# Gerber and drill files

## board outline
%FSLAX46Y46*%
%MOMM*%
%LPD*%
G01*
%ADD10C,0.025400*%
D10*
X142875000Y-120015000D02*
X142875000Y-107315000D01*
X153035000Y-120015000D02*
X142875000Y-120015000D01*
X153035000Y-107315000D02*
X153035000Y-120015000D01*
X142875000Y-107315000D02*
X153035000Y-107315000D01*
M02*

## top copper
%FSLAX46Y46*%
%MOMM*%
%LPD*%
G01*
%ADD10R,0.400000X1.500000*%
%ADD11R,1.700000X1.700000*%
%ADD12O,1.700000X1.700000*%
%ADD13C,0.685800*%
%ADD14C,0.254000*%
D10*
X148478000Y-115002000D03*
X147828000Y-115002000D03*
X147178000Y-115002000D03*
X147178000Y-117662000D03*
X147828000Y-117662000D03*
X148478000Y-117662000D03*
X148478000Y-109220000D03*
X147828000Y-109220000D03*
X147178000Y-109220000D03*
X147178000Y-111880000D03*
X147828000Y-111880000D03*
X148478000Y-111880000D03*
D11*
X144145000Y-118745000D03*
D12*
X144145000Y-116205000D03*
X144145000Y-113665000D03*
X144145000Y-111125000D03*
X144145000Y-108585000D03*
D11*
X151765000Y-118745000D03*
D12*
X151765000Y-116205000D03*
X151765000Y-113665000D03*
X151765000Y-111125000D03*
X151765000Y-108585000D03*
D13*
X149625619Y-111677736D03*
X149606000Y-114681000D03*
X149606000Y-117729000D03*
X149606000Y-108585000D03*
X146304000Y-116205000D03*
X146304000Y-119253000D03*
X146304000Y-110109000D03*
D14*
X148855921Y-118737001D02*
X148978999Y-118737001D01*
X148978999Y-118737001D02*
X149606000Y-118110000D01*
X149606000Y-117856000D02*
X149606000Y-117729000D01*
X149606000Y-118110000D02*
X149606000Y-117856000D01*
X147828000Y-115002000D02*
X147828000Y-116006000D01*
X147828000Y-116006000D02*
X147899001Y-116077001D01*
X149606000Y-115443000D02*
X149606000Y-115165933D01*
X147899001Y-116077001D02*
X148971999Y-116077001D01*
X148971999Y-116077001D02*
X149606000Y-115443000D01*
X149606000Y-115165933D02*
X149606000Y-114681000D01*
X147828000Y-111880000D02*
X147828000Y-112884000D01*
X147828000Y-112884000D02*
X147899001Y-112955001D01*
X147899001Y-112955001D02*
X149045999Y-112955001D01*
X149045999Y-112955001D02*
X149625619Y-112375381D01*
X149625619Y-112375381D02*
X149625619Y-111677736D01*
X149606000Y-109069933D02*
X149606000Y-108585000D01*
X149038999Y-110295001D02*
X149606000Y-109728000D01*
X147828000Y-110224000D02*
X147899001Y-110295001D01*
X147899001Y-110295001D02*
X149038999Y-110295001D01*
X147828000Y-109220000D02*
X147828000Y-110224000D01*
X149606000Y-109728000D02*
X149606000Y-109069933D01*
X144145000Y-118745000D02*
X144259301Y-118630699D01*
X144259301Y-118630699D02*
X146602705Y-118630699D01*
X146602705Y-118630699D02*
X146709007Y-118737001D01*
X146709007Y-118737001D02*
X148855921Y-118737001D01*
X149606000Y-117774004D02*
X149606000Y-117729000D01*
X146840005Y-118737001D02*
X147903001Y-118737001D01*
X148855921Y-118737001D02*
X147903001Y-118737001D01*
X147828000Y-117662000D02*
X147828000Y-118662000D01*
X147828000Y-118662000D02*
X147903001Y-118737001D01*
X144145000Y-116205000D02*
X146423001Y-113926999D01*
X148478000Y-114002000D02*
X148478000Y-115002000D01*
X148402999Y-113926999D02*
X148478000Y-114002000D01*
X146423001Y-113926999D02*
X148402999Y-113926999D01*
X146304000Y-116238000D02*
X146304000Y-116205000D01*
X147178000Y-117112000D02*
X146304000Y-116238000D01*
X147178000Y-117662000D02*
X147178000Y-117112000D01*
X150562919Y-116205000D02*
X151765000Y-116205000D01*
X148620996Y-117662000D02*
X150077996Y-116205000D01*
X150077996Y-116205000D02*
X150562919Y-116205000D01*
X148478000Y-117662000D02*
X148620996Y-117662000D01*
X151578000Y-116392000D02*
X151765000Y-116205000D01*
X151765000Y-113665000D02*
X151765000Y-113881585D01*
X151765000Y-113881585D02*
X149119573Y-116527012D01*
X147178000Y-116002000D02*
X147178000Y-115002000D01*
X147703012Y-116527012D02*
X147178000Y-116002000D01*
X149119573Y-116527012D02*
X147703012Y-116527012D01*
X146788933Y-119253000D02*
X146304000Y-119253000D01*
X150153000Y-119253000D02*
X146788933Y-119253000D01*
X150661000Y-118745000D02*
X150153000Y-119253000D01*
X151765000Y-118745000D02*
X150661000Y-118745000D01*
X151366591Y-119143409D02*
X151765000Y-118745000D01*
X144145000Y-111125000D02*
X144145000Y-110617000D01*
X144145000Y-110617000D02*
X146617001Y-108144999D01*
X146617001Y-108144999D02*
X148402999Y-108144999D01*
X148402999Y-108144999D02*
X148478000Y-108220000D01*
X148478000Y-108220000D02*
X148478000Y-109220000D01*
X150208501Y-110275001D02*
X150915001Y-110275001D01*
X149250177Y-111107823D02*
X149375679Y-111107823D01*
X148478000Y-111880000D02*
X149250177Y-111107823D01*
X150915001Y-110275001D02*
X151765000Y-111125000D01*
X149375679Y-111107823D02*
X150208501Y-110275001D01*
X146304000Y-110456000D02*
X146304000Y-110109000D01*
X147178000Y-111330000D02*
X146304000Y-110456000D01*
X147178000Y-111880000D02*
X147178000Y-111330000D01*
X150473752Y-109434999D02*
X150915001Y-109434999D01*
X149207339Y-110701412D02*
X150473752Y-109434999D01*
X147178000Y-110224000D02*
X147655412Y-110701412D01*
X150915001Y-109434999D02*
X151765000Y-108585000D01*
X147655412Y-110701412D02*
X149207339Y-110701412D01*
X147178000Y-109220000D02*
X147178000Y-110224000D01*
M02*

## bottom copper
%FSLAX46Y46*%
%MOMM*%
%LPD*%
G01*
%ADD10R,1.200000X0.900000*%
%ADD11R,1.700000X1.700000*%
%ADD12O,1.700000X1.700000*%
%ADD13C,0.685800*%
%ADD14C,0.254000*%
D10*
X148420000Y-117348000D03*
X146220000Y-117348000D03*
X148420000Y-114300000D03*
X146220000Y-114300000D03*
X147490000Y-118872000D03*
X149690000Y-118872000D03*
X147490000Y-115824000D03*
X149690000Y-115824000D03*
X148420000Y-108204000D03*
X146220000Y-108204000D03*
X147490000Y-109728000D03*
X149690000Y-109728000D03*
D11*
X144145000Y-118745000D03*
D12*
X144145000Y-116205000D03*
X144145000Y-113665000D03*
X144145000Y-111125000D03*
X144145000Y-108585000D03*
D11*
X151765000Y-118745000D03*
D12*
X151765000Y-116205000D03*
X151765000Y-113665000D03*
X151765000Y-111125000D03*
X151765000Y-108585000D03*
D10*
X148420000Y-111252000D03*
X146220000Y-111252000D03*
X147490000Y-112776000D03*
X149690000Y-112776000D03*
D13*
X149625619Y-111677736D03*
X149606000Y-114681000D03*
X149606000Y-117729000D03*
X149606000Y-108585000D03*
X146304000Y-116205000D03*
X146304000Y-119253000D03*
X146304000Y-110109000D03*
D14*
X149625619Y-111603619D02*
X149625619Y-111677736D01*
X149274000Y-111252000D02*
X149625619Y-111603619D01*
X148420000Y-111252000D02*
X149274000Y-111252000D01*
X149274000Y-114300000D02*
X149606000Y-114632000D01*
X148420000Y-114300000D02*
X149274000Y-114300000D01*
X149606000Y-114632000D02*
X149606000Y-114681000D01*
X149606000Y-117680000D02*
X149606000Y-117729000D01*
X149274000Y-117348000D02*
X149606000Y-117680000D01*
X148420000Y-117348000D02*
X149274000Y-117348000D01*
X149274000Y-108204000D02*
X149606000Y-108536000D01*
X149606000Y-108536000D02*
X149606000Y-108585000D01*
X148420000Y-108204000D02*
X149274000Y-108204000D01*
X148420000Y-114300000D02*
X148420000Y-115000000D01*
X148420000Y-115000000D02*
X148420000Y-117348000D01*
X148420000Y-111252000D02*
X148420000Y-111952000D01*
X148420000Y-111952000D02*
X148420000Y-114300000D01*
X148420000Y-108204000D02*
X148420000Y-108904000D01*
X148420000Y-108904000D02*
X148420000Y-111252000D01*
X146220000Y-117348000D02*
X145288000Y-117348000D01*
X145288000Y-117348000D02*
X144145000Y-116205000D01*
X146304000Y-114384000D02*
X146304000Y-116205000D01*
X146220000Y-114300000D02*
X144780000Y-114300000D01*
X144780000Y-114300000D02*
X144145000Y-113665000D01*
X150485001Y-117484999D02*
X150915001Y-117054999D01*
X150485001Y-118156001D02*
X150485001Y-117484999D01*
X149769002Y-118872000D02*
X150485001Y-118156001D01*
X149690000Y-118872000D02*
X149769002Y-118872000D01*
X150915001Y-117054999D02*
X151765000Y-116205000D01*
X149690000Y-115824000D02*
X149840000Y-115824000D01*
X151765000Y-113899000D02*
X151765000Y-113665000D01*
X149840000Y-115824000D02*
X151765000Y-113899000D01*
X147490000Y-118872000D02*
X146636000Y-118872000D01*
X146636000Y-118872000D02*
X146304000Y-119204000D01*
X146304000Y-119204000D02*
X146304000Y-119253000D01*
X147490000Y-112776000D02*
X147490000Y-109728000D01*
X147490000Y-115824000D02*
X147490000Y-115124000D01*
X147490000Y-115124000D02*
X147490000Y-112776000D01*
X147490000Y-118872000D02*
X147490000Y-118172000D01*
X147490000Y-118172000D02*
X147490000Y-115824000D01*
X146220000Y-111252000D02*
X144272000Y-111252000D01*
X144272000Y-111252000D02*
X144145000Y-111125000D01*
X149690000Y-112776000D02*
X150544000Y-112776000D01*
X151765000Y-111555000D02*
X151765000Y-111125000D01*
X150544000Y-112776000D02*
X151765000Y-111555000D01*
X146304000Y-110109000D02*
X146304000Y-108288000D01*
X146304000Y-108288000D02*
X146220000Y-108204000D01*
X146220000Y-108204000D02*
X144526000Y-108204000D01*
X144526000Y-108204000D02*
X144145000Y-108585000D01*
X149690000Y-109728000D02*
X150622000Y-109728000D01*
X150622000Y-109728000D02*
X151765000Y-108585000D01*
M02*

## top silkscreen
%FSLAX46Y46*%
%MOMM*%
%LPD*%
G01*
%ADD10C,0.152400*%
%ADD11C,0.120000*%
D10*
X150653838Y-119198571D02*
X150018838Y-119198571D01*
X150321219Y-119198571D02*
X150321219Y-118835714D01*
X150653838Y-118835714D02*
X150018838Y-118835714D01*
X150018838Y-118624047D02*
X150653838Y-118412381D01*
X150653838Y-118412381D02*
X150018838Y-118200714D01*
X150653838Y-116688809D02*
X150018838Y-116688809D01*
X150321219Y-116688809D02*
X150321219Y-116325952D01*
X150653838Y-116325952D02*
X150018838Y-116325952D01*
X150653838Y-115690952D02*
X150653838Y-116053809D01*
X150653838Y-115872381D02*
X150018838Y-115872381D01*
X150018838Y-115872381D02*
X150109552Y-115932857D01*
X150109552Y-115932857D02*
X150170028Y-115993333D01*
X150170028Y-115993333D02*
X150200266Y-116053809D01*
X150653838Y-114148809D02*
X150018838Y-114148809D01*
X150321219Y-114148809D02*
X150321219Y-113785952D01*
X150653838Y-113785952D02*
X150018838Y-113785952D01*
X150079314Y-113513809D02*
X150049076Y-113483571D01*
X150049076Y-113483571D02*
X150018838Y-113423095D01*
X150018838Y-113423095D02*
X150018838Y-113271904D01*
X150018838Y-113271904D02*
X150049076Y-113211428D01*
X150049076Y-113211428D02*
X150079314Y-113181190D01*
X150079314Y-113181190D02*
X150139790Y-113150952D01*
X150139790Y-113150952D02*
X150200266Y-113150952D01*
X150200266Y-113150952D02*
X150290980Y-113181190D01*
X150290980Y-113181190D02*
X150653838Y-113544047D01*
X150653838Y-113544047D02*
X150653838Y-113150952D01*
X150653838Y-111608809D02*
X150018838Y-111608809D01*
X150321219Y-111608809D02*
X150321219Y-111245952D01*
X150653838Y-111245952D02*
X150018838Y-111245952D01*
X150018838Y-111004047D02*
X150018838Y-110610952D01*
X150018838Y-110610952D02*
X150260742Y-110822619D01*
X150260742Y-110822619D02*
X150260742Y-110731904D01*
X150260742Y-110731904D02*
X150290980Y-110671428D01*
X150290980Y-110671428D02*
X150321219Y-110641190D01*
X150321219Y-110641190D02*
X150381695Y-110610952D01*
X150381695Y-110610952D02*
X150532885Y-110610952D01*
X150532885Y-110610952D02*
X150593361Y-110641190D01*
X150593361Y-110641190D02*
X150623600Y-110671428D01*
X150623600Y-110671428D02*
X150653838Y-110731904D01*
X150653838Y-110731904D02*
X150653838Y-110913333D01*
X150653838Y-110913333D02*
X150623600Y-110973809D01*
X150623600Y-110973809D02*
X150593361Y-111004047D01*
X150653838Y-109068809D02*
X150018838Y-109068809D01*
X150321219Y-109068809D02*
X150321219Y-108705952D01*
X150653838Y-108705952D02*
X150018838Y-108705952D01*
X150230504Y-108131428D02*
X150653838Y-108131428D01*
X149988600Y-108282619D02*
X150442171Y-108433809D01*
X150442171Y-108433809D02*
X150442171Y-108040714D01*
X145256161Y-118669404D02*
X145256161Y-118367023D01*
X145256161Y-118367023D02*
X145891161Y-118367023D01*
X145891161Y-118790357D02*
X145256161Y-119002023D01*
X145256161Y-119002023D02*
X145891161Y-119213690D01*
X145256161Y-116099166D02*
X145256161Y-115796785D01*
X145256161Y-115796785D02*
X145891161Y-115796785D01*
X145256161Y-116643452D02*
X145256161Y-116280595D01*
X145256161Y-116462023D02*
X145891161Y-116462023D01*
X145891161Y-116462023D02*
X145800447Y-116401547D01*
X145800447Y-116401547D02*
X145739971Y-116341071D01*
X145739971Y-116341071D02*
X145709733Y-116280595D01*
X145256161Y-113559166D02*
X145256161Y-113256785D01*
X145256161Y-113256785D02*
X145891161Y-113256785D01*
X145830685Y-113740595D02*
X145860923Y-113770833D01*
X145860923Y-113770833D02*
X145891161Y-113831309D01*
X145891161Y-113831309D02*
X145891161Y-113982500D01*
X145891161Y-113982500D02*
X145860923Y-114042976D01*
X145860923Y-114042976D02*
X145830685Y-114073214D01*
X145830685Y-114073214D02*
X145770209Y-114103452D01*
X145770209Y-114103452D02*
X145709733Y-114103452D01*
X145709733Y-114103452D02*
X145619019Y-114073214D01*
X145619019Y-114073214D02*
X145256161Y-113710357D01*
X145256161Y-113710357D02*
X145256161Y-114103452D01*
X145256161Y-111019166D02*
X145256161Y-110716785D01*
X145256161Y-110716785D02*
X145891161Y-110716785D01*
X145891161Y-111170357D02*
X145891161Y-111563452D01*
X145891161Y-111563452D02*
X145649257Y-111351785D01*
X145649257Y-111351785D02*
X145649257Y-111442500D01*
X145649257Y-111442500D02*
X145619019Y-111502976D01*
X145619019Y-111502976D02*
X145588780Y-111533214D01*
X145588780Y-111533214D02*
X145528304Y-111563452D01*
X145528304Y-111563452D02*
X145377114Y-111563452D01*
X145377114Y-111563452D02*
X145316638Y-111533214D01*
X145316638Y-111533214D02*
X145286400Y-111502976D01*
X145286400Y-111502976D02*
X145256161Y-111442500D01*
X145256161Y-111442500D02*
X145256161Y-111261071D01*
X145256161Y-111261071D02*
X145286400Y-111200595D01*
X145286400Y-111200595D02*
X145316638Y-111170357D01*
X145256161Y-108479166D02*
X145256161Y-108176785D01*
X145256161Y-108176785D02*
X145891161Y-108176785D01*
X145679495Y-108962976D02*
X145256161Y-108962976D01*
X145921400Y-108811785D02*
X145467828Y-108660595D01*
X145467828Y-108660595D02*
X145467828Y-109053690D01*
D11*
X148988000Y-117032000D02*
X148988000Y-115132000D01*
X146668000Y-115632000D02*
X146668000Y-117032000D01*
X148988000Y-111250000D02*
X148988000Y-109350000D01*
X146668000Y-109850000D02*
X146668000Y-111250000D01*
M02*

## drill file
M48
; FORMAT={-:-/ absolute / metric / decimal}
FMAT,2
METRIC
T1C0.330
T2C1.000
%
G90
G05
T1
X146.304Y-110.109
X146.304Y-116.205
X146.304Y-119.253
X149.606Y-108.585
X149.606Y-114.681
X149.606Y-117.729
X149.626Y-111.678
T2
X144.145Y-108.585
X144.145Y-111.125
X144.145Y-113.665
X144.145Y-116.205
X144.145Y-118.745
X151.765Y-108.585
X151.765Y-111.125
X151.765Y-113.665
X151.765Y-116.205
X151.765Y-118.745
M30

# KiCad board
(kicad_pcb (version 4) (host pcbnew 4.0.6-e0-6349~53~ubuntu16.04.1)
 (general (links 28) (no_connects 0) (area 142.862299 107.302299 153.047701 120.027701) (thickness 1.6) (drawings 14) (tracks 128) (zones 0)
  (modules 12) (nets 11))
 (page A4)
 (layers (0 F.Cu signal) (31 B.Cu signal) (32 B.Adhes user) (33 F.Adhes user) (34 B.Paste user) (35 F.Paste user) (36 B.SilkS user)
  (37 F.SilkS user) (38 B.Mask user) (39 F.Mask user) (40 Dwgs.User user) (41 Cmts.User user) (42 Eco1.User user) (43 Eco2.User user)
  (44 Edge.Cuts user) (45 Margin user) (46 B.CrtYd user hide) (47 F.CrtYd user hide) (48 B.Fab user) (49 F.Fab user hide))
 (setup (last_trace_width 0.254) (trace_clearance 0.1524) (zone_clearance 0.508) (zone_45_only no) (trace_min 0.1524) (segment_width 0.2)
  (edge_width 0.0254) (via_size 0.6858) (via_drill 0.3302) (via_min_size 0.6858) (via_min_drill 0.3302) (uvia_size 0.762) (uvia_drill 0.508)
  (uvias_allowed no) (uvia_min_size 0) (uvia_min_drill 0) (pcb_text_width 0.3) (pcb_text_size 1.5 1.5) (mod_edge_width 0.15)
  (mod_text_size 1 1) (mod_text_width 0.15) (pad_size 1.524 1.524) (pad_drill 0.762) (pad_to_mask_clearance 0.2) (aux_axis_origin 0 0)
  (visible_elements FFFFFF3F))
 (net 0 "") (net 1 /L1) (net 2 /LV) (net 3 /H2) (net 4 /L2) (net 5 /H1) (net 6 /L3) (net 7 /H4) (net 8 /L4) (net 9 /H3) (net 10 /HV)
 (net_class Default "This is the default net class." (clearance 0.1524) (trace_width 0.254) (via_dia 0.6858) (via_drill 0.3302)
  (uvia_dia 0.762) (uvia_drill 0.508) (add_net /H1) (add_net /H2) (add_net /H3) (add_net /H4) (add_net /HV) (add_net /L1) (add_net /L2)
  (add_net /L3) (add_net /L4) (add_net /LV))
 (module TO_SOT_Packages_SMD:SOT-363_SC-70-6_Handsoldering (layer F.Cu) (at 147.828 116.332 270)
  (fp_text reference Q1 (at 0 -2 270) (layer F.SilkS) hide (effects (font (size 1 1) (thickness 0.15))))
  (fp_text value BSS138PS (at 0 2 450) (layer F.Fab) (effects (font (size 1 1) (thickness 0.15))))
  (fp_line (start 0.7 -1.16) (end -1.2 -1.16) (layer F.SilkS) (width 0.12))
  (fp_line (start -0.7 1.16) (end 0.7 1.16) (layer F.SilkS) (width 0.12))
  (pad 1 smd rect (at -1.33 -0.65 270) (size 1.5 0.4) (layers F.Cu F.Paste F.Mask) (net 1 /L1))
  (pad 2 smd rect (at -1.33 0 270) (size 1.5 0.4) (layers F.Cu F.Paste F.Mask) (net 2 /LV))
  (pad 3 smd rect (at -1.33 0.65 270) (size 1.5 0.4) (layers F.Cu F.Paste F.Mask) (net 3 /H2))
  (pad 4 smd rect (at 1.33 0.65 270) (size 1.5 0.4) (layers F.Cu F.Paste F.Mask) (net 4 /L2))
  (pad 5 smd rect (at 1.33 0 270) (size 1.5 0.4) (layers F.Cu F.Paste F.Mask) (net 2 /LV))
  (pad 6 smd rect (at 1.33 -0.65 270) (size 1.5 0.4) (layers F.Cu F.Paste F.Mask) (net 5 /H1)))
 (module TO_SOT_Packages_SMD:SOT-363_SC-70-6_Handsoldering (layer F.Cu) (at 147.828 110.55 270)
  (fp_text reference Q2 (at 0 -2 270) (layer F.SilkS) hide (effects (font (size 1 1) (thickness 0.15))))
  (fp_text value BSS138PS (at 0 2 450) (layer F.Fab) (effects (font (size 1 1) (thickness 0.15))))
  (fp_line (start 0.7 -1.16) (end -1.2 -1.16) (layer F.SilkS) (width 0.12))
  (fp_line (start -0.7 1.16) (end 0.7 1.16) (layer F.SilkS) (width 0.12))
  (pad 1 smd rect (at -1.33 -0.65 270) (size 1.5 0.4) (layers F.Cu F.Paste F.Mask) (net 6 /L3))
  (pad 2 smd rect (at -1.33 0 270) (size 1.5 0.4) (layers F.Cu F.Paste F.Mask) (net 2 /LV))
  (pad 3 smd rect (at -1.33 0.65 270) (size 1.5 0.4) (layers F.Cu F.Paste F.Mask) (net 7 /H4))
  (pad 4 smd rect (at 1.33 0.65 270) (size 1.5 0.4) (layers F.Cu F.Paste F.Mask) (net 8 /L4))
  (pad 5 smd rect (at 1.33 0 270) (size 1.5 0.4) (layers F.Cu F.Paste F.Mask) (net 2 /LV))
  (pad 6 smd rect (at 1.33 -0.65 270) (size 1.5 0.4) (layers F.Cu F.Paste F.Mask) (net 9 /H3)))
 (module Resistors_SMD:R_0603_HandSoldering (layer B.Cu) (at 147.32 117.348 180)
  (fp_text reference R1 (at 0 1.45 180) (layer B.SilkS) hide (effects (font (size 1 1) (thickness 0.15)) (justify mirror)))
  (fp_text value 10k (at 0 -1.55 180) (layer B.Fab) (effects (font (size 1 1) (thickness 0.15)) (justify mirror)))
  (pad 1 smd rect (at -1.1 0 180) (size 1.2 0.9) (layers B.Cu B.Paste B.Mask) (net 2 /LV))
  (pad 2 smd rect (at 1.1 0 180) (size 1.2 0.9) (layers B.Cu B.Paste B.Mask) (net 1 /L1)))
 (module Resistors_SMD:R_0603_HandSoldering (layer B.Cu) (at 147.32 114.3 180)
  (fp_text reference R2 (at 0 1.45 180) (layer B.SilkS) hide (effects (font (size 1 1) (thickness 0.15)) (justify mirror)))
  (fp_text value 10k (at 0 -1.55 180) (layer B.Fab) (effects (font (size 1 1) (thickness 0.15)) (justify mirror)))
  (pad 1 smd rect (at -1.1 0 180) (size 1.2 0.9) (layers B.Cu B.Paste B.Mask) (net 2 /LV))
  (pad 2 smd rect (at 1.1 0 180) (size 1.2 0.9) (layers B.Cu B.Paste B.Mask) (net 4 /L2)))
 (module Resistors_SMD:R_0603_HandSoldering (layer B.Cu) (at 148.59 118.872)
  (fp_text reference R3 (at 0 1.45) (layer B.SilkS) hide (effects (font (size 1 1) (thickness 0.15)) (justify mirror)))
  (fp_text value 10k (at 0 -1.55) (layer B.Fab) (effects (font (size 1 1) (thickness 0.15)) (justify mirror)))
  (pad 1 smd rect (at -1.1 0) (size 1.2 0.9) (layers B.Cu B.Paste B.Mask) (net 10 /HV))
  (pad 2 smd rect (at 1.1 0) (size 1.2 0.9) (layers B.Cu B.Paste B.Mask) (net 5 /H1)))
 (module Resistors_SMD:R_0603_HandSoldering (layer B.Cu) (at 148.59 115.824)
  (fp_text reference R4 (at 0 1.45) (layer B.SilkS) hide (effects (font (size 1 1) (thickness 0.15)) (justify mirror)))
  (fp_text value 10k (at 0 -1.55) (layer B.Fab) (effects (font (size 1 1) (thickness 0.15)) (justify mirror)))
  (pad 1 smd rect (at -1.1 0) (size 1.2 0.9) (layers B.Cu B.Paste B.Mask) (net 10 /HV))
  (pad 2 smd rect (at 1.1 0) (size 1.2 0.9) (layers B.Cu B.Paste B.Mask) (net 3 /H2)))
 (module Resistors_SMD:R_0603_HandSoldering (layer B.Cu) (at 147.32 108.204 180)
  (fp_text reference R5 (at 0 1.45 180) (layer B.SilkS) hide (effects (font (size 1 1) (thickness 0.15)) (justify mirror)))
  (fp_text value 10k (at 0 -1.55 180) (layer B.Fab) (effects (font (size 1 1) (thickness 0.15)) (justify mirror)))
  (pad 1 smd rect (at -1.1 0 180) (size 1.2 0.9) (layers B.Cu B.Paste B.Mask) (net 2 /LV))
  (pad 2 smd rect (at 1.1 0 180) (size 1.2 0.9) (layers B.Cu B.Paste B.Mask) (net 8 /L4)))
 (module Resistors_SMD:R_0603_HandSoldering (layer B.Cu) (at 148.59 109.728)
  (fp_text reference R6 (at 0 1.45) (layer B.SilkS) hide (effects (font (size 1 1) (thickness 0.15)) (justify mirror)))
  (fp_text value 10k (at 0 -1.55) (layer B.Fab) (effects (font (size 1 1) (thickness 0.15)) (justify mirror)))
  (pad 1 smd rect (at -1.1 0) (size 1.2 0.9) (layers B.Cu B.Paste B.Mask) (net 10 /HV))
  (pad 2 smd rect (at 1.1 0) (size 1.2 0.9) (layers B.Cu B.Paste B.Mask) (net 7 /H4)))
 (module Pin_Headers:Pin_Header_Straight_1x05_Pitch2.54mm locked (layer B.Cu) (at 144.145 118.745)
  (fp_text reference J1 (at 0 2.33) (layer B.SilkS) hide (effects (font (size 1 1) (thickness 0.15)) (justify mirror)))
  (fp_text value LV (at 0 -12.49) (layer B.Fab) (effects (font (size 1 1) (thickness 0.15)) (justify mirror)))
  (pad 1 thru_hole rect (at 0 0) (size 1.7 1.7) (drill 1) (layers *.Cu *.Mask) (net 2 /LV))
  (pad 2 thru_hole oval (at 0 -2.54) (size 1.7 1.7) (drill 1) (layers *.Cu *.Mask) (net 1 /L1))
  (pad 3 thru_hole oval (at 0 -5.08) (size 1.7 1.7) (drill 1) (layers *.Cu *.Mask) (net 4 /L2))
  (pad 4 thru_hole oval (at 0 -7.62) (size 1.7 1.7) (drill 1) (layers *.Cu *.Mask) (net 6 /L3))
  (pad 5 thru_hole oval (at 0 -10.16) (size 1.7 1.7) (drill 1) (layers *.Cu *.Mask) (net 8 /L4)))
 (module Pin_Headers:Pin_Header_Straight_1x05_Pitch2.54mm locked (layer B.Cu) (at 151.765 118.745)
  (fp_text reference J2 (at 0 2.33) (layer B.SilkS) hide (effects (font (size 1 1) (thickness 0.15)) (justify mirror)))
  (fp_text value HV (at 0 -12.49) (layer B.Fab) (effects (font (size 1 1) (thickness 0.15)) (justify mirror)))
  (pad 1 thru_hole rect (at 0 0) (size 1.7 1.7) (drill 1) (layers *.Cu *.Mask) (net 10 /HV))
  (pad 2 thru_hole oval (at 0 -2.54) (size 1.7 1.7) (drill 1) (layers *.Cu *.Mask) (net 5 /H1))
  (pad 3 thru_hole oval (at 0 -5.08) (size 1.7 1.7) (drill 1) (layers *.Cu *.Mask) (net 3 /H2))
  (pad 4 thru_hole oval (at 0 -7.62) (size 1.7 1.7) (drill 1) (layers *.Cu *.Mask) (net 9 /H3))
  (pad 5 thru_hole oval (at 0 -10.16) (size 1.7 1.7) (drill 1) (layers *.Cu *.Mask) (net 7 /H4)))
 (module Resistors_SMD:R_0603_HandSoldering (layer B.Cu) (at 147.32 111.252 180)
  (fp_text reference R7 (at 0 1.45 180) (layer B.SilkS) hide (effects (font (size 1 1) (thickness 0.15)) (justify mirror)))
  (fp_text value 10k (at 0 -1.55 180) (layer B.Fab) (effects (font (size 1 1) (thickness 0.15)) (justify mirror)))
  (pad 1 smd rect (at -1.1 0 180) (size 1.2 0.9) (layers B.Cu B.Paste B.Mask) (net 2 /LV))
  (pad 2 smd rect (at 1.1 0 180) (size 1.2 0.9) (layers B.Cu B.Paste B.Mask) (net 6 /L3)))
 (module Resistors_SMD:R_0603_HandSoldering (layer B.Cu) (at 148.59 112.776)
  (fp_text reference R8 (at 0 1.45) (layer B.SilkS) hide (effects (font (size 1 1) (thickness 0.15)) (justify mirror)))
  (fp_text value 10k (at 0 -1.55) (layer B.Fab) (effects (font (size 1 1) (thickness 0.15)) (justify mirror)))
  (pad 1 smd rect (at -1.1 0) (size 1.2 0.9) (layers B.Cu B.Paste B.Mask) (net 10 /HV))
  (pad 2 smd rect (at 1.1 0) (size 1.2 0.9) (layers B.Cu B.Paste B.Mask) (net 9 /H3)))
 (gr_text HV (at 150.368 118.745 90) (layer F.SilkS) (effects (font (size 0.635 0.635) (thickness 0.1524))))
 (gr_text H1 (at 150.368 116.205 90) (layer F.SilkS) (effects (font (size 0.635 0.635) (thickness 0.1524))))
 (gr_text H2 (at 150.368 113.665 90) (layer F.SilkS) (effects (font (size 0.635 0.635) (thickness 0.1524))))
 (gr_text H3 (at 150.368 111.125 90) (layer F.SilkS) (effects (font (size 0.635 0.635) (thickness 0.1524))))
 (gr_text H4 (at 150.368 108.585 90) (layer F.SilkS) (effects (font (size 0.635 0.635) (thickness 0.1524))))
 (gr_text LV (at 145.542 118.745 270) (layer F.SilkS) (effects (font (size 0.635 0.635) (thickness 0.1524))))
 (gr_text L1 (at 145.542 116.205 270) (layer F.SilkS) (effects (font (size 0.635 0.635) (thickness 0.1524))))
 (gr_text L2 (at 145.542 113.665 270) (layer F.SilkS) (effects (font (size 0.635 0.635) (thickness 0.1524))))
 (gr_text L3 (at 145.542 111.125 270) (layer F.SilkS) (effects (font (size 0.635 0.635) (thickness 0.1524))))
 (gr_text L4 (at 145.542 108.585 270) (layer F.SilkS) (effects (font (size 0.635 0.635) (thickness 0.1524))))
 (gr_line (start 142.875 120.015) (end 142.875 107.315) (angle 90) (layer Edge.Cuts) (width 0.0254))
 (gr_line (start 153.035 120.015) (end 142.875 120.015) (angle 90) (layer Edge.Cuts) (width 0.0254))
 (gr_line (start 153.035 107.315) (end 153.035 120.015) (angle 90) (layer Edge.Cuts) (width 0.0254))
 (gr_line (start 142.875 107.315) (end 153.035 107.315) (angle 90) (layer Edge.Cuts) (width 0.0254))
 (segment (start 148.855921 118.737001) (end 148.978999 118.737001) (width 0.254) (layer F.Cu) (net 2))
 (segment (start 148.978999 118.737001) (end 149.606 118.11) (width 0.254) (layer F.Cu) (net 2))
 (segment (start 149.606 117.856) (end 149.606 117.729) (width 0.254) (layer F.Cu) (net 2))
 (segment (start 149.606 118.11) (end 149.606 117.856) (width 0.254) (layer F.Cu) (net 2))
 (segment (start 147.828 115.002) (end 147.828 116.006) (width 0.254) (layer F.Cu) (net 2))
 (segment (start 147.828 116.006) (end 147.899001 116.077001) (width 0.254) (layer F.Cu) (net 2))
 (segment (start 149.606 115.443) (end 149.606 115.165933) (width 0.254) (layer F.Cu) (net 2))
 (segment (start 147.899001 116.077001) (end 148.971999 116.077001) (width 0.254) (layer F.Cu) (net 2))
 (segment (start 148.971999 116.077001) (end 149.606 115.443) (width 0.254) (layer F.Cu) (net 2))
 (segment (start 149.606 115.165933) (end 149.606 114.681) (width 0.254) (layer F.Cu) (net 2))
 (segment (start 147.828 111.88) (end 147.828 112.884) (width 0.254) (layer F.Cu) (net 2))
 (segment (start 147.828 112.884) (end 147.899001 112.955001) (width 0.254) (layer F.Cu) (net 2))
 (segment (start 147.899001 112.955001) (end 149.045999 112.955001) (width 0.254) (layer F.Cu) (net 2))
 (segment (start 149.045999 112.955001) (end 149.625619 112.375381) (width 0.254) (layer F.Cu) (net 2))
 (segment (start 149.625619 112.375381) (end 149.625619 111.677736) (width 0.254) (layer F.Cu) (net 2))
 (segment (start 149.625619 111.603619) (end 149.625619 111.677736) (width 0.254) (layer B.Cu) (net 2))
 (segment (start 149.606 109.069933) (end 149.606 108.585) (width 0.254) (layer F.Cu) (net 2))
 (segment (start 149.274 111.252) (end 149.625619 111.603619) (width 0.254) (layer B.Cu) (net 2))
 (segment (start 149.038999 110.295001) (end 149.606 109.728) (width 0.254) (layer F.Cu) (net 2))
 (segment (start 148.42 111.252) (end 149.274 111.252) (width 0.254) (layer B.Cu) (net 2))
 (segment (start 147.828 110.224) (end 147.899001 110.295001) (width 0.254) (layer F.Cu) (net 2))
 (segment (start 147.899001 110.295001) (end 149.038999 110.295001) (width 0.254) (layer F.Cu) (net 2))
 (via (at 149.625619 111.677736) (size 0.6858) (drill 0.3302) (layers F.Cu B.Cu) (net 2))
 (segment (start 147.828 109.22) (end 147.828 110.224) (width 0.254) (layer F.Cu) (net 2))
 (segment (start 149.606 109.728) (end 149.606 109.069933) (width 0.254) (layer F.Cu) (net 2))
 (segment (start 144.145 118.745) (end 144.259301 118.630699) (width 0.254) (layer F.Cu) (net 2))
 (segment (start 144.259301 118.630699) (end 146.602705 118.630699) (width 0.254) (layer F.Cu) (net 2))
 (segment (start 146.602705 118.630699) (end 146.709007 118.737001) (width 0.254) (layer F.Cu) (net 2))
 (segment (start 146.709007 118.737001) (end 148.855921 118.737001) (width 0.254) (layer F.Cu) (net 2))
 (segment (start 149.274 114.3) (end 149.606 114.632) (width 0.254) (layer B.Cu) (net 2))
 (segment (start 148.42 114.3) (end 149.274 114.3) (width 0.254) (layer B.Cu) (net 2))
 (segment (start 149.606 114.632) (end 149.606 114.681) (width 0.254) (layer B.Cu) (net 2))
 (via (at 149.606 114.681) (size 0.6858) (drill 0.3302) (layers F.Cu B.Cu) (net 2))
 (segment (start 149.606 117.68) (end 149.606 117.729) (width 0.254) (layer B.Cu) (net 2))
 (segment (start 149.274 117.348) (end 149.606 117.68) (width 0.254) (layer B.Cu) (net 2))
 (segment (start 149.606 117.774004) (end 149.606 117.729) (width 0.254) (layer F.Cu) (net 2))
 (segment (start 148.42 117.348) (end 149.274 117.348) (width 0.254) (layer B.Cu) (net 2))
 (via (at 149.606 117.729) (size 0.6858) (drill 0.3302) (layers F.Cu B.Cu) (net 2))
 (segment (start 149.274 108.204) (end 149.606 108.536) (width 0.254) (layer B.Cu) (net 2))
 (segment (start 149.606 108.536) (end 149.606 108.585) (width 0.254) (layer B.Cu) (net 2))
 (segment (start 148.42 108.204) (end 149.274 108.204) (width 0.254) (layer B.Cu) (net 2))
 (via (at 149.606 108.585) (size 0.6858) (drill 0.3302) (layers F.Cu B.Cu) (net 2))
 (segment (start 146.840005 118.737001) (end 147.903001 118.737001) (width 0.254) (layer F.Cu) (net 2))
 (segment (start 148.855921 118.737001) (end 147.903001 118.737001) (width 0.254) (layer F.Cu) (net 2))
 (segment (start 147.828 117.662) (end 147.828 118.662) (width 0.254) (layer F.Cu) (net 2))
 (segment (start 147.828 118.662) (end 147.903001 118.737001) (width 0.254) (layer F.Cu) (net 2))
 (segment (start 148.42 114.3) (end 148.42 115) (width 0.254) (layer B.Cu) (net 2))
 (segment (start 148.42 115) (end 148.42 117.348) (width 0.254) (layer B.Cu) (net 2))
 (segment (start 148.42 111.252) (end 148.42 111.952) (width 0.254) (layer B.Cu) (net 2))
 (segment (start 148.42 111.952) (end 148.42 114.3) (width 0.254) (layer B.Cu) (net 2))
 (segment (start 148.42 108.204) (end 148.42 108.904) (width 0.254) (layer B.Cu) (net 2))
 (segment (start 148.42 108.904) (end 148.42 111.252) (width 0.254) (layer B.Cu) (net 2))
 (segment (start 144.145 116.205) (end 146.423001 113.926999) (width 0.254) (layer F.Cu) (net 1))
 (segment (start 148.478 114.002) (end 148.478 115.002) (width 0.254) (layer F.Cu) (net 1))
 (segment (start 148.402999 113.926999) (end 148.478 114.002) (width 0.254) (layer F.Cu) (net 1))
 (segment (start 146.423001 113.926999) (end 148.402999 113.926999) (width 0.254) (layer F.Cu) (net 1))
 (segment (start 146.22 117.348) (end 145.288 117.348) (width 0.254) (layer B.Cu) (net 1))
 (segment (start 145.288 117.348) (end 144.145 116.205) (width 0.254) (layer B.Cu) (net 1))
 (segment (start 146.304 116.238) (end 146.304 116.205) (width 0.254) (layer F.Cu) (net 4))
 (segment (start 147.178 117.112) (end 146.304 116.238) (width 0.254) (layer F.Cu) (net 4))
 (segment (start 147.178 117.662) (end 147.178 117.112) (width 0.254) (layer F.Cu) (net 4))
 (segment (start 146.304 114.384) (end 146.304 116.205) (width 0.254) (layer B.Cu) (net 4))
 (via (at 146.304 116.205) (size 0.6858) (drill 0.3302) (layers F.Cu B.Cu) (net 4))
 (segment (start 146.22 114.3) (end 144.78 114.3) (width 0.254) (layer B.Cu) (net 4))
 (segment (start 144.78 114.3) (end 144.145 113.665) (width 0.254) (layer B.Cu) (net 4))
 (segment (start 150.562919 116.205) (end 151.765 116.205) (width 0.254) (layer F.Cu) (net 5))
 (segment (start 148.620996 117.662) (end 150.077996 116.205) (width 0.254) (layer F.Cu) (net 5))
 (segment (start 150.077996 116.205) (end 150.562919 116.205) (width 0.254) (layer F.Cu) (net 5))
 (segment (start 148.478 117.662) (end 148.620996 117.662) (width 0.254) (layer F.Cu) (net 5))
 (segment (start 150.485001 117.484999) (end 150.915001 117.054999) (width 0.254) (layer B.Cu) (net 5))
 (segment (start 150.485001 118.156001) (end 150.485001 117.484999) (width 0.254) (layer B.Cu) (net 5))
 (segment (start 149.769002 118.872) (end 150.485001 118.156001) (width 0.254) (layer B.Cu) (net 5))
 (segment (start 149.69 118.872) (end 149.769002 118.872) (width 0.254) (layer B.Cu) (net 5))
 (segment (start 150.915001 117.054999) (end 151.765 116.205) (width 0.254) (layer B.Cu) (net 5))
 (segment (start 151.578 116.392) (end 151.765 116.205) (width 0.254) (layer F.Cu) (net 5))
 (segment (start 151.765 113.665) (end 151.765 113.881585) (width 0.254) (layer F.Cu) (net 3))
 (segment (start 151.765 113.881585) (end 149.119573 116.527012) (width 0.254) (layer F.Cu) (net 3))
 (segment (start 147.178 116.002) (end 147.178 115.002) (width 0.254) (layer F.Cu) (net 3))
 (segment (start 147.703012 116.527012) (end 147.178 116.002) (width 0.254) (layer F.Cu) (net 3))
 (segment (start 149.119573 116.527012) (end 147.703012 116.527012) (width 0.254) (layer F.Cu) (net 3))
 (segment (start 149.69 115.824) (end 149.84 115.824) (width 0.254) (layer B.Cu) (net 3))
 (segment (start 151.765 113.899) (end 151.765 113.665) (width 0.254) (layer B.Cu) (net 3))
 (segment (start 149.84 115.824) (end 151.765 113.899) (width 0.254) (layer B.Cu) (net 3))
 (segment (start 146.788933 119.253) (end 146.304 119.253) (width 0.254) (layer F.Cu) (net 10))
 (segment (start 150.153 119.253) (end 146.788933 119.253) (width 0.254) (layer F.Cu) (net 10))
 (segment (start 150.661 118.745) (end 150.153 119.253) (width 0.254) (layer F.Cu) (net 10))
 (segment (start 151.765 118.745) (end 150.661 118.745) (width 0.254) (layer F.Cu) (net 10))
 (segment (start 147.49 118.872) (end 146.636 118.872) (width 0.254) (layer B.Cu) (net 10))
 (via (at 146.304 119.253) (size 0.6858) (drill 0.3302) (layers F.Cu B.Cu) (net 10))
 (segment (start 146.636 118.872) (end 146.304 119.204) (width 0.254) (layer B.Cu) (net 10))
 (segment (start 146.304 119.204) (end 146.304 119.253) (width 0.254) (layer B.Cu) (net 10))
 (segment (start 151.366591 119.143409) (end 151.765 118.745) (width 0.254) (layer F.Cu) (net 10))
 (segment (start 147.49 112.776) (end 147.49 109.728) (width 0.254) (layer B.Cu) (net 10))
 (segment (start 147.49 115.824) (end 147.49 115.124) (width 0.254) (layer B.Cu) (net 10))
 (segment (start 147.49 115.124) (end 147.49 112.776) (width 0.254) (layer B.Cu) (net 10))
 (segment (start 147.49 118.872) (end 147.49 118.172) (width 0.254) (layer B.Cu) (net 10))
 (segment (start 147.49 118.172) (end 147.49 115.824) (width 0.254) (layer B.Cu) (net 10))
 (segment (start 144.145 111.125) (end 144.145 110.617) (width 0.254) (layer F.Cu) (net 6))
 (segment (start 144.145 110.617) (end 146.617001 108.144999) (width 0.254) (layer F.Cu) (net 6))
 (segment (start 146.617001 108.144999) (end 148.402999 108.144999) (width 0.254) (layer F.Cu) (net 6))
 (segment (start 148.402999 108.144999) (end 148.478 108.22) (width 0.254) (layer F.Cu) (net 6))
 (segment (start 148.478 108.22) (end 148.478 109.22) (width 0.254) (layer F.Cu) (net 6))
 (segment (start 146.22 111.252) (end 144.272 111.252) (width 0.254) (layer B.Cu) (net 6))
 (segment (start 144.272 111.252) (end 144.145 111.125) (width 0.254) (layer B.Cu) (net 6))
 (segment (start 150.208501 110.275001) (end 150.915001 110.275001) (width 0.254) (layer F.Cu) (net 9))
 (segment (start 149.250177 111.107823) (end 149.375679 111.107823) (width 0.254) (layer F.Cu) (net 9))
 (segment (start 148.478 111.88) (end 149.250177 111.107823) (width 0.254) (layer F.Cu) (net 9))
 (segment (start 150.915001 110.275001) (end 151.765 111.125) (width 0.254) (layer F.Cu) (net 9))
 (segment (start 149.375679 111.107823) (end 150.208501 110.275001) (width 0.254) (layer F.Cu) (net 9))
 (segment (start 149.69 112.776) (end 150.544 112.776) (width 0.254) (layer B.Cu) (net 9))
 (segment (start 151.765 111.555) (end 151.765 111.125) (width 0.254) (layer B.Cu) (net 9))
 (segment (start 150.544 112.776) (end 151.765 111.555) (width 0.254) (layer B.Cu) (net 9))
 (segment (start 146.304 110.109) (end 146.304 108.288) (width 0.254) (layer B.Cu) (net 8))
 (segment (start 146.304 108.288) (end 146.22 108.204) (width 0.254) (layer B.Cu) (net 8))
 (segment (start 146.304 110.456) (end 146.304 110.109) (width 0.254) (layer F.Cu) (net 8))
 (segment (start 147.178 111.33) (end 146.304 110.456) (width 0.254) (layer F.Cu) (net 8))
 (segment (start 147.178 111.88) (end 147.178 111.33) (width 0.254) (layer F.Cu) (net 8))
 (via (at 146.304 110.109) (size 0.6858) (drill 0.3302) (layers F.Cu B.Cu) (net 8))
 (segment (start 146.22 108.204) (end 144.526 108.204) (width 0.254) (layer B.Cu) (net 8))
 (segment (start 144.526 108.204) (end 144.145 108.585) (width 0.254) (layer B.Cu) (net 8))
 (segment (start 150.473752 109.434999) (end 150.915001 109.434999) (width 0.254) (layer F.Cu) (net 7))
 (segment (start 149.207339 110.701412) (end 150.473752 109.434999) (width 0.254) (layer F.Cu) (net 7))
 (segment (start 147.178 110.224) (end 147.655412 110.701412) (width 0.254) (layer F.Cu) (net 7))
 (segment (start 150.915001 109.434999) (end 151.765 108.585) (width 0.254) (layer F.Cu) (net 7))
 (segment (start 147.655412 110.701412) (end 149.207339 110.701412) (width 0.254) (layer F.Cu) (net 7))
 (segment (start 147.178 109.22) (end 147.178 110.224) (width 0.254) (layer F.Cu) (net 7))
 (segment (start 149.69 109.728) (end 150.622 109.728) (width 0.254) (layer B.Cu) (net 7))
 (segment (start 150.622 109.728) (end 151.765 108.585) (width 0.254) (layer B.Cu) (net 7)))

